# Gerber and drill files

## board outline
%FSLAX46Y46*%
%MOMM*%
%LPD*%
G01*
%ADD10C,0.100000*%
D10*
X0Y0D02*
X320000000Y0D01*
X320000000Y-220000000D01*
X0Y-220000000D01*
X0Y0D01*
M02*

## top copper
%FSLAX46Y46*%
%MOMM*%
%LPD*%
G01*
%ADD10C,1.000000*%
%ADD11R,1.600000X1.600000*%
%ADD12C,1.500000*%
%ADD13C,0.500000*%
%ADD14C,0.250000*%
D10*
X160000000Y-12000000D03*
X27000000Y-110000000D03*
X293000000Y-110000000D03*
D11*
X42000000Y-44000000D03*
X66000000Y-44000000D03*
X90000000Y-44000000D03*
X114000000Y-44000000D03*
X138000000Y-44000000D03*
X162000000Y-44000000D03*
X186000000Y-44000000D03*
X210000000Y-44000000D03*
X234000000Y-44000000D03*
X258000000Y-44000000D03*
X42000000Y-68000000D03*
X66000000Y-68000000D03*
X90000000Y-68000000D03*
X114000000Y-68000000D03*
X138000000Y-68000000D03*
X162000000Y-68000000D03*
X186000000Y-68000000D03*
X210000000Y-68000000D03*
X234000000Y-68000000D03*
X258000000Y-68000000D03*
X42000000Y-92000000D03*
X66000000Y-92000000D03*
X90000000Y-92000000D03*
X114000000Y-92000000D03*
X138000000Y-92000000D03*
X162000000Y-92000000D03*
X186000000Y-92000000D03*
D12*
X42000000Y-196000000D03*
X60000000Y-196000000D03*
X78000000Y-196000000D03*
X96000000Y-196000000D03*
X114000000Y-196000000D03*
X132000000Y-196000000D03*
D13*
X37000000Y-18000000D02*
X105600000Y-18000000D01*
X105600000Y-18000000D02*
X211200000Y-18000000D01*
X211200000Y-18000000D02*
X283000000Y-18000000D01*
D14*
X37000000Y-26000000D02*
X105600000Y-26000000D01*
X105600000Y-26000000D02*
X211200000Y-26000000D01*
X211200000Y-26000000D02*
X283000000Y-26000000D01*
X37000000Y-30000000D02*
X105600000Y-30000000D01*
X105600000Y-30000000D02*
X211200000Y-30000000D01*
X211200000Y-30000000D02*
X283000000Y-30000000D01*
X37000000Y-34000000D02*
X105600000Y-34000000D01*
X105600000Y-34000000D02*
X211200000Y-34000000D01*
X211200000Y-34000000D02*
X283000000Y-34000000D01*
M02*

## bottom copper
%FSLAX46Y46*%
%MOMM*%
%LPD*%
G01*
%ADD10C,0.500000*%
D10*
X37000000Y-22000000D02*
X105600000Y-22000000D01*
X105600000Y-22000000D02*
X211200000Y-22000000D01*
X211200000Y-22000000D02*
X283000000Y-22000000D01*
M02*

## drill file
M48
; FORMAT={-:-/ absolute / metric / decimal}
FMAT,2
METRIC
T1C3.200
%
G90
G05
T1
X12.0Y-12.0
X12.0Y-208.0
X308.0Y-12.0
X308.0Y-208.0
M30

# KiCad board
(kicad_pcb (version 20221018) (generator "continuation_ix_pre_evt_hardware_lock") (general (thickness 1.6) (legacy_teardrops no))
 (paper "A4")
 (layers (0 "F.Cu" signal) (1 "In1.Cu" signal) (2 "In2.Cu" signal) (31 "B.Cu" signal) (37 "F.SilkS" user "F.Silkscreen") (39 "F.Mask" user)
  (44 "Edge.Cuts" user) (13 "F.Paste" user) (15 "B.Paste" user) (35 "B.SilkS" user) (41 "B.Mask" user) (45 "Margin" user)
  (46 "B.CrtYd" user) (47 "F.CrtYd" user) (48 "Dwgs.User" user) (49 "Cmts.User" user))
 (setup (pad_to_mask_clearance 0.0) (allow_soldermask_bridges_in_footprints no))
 (gr_rect (start 0 0) (end 320.0 220.0) (stroke (width 0.1) (type default)) (fill none) (layer "Edge.Cuts"))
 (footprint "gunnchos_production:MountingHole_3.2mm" (layer "F.Cu") (at 12.0 12.0)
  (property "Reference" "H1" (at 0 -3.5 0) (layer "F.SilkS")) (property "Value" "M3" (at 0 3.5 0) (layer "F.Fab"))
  (pad "" np_thru_hole circle (at 0 0) (size 3.2 3.2) (drill 3.2) (layers "*.Cu" "*.Mask")))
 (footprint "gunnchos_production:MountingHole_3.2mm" (layer "F.Cu") (at 308.0 12.0)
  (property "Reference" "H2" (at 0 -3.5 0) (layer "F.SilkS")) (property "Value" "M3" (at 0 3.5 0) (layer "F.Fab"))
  (pad "" np_thru_hole circle (at 0 0) (size 3.2 3.2) (drill 3.2) (layers "*.Cu" "*.Mask")))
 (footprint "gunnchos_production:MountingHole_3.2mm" (layer "F.Cu") (at 12.0 208.0)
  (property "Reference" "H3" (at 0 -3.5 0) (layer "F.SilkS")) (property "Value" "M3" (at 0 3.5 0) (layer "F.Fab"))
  (pad "" np_thru_hole circle (at 0 0) (size 3.2 3.2) (drill 3.2) (layers "*.Cu" "*.Mask")))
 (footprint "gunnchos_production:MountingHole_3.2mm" (layer "F.Cu") (at 308.0 208.0)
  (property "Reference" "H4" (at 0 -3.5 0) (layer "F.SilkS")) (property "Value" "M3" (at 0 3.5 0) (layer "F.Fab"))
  (pad "" np_thru_hole circle (at 0 0) (size 3.2 3.2) (drill 3.2) (layers "*.Cu" "*.Mask")))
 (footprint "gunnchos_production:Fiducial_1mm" (layer "F.Cu") (at 160.0 12.0)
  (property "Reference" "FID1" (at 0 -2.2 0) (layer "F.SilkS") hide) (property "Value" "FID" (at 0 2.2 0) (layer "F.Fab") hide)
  (pad "1" smd circle (at 0 0) (size 1 1) (layers "F.Cu") (solder_mask_margin 0.5)))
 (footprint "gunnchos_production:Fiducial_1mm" (layer "F.Cu") (at 27.0 110.0)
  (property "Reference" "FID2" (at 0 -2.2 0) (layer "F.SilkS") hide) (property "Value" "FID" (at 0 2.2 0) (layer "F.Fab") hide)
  (pad "1" smd circle (at 0 0) (size 1 1) (layers "F.Cu") (solder_mask_margin 0.5)))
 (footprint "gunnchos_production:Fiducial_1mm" (layer "F.Cu") (at 293.0 110.0)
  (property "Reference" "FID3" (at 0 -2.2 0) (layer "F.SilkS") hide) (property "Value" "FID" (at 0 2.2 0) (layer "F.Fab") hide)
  (pad "1" smd circle (at 0 0) (size 1 1) (layers "F.Cu") (solder_mask_margin 0.5)))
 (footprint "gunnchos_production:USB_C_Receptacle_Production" (layer "F.Cu") (at 42.00 44.00)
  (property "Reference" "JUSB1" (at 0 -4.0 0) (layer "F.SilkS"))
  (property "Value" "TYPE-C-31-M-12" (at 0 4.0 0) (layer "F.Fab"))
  (pad "1" smd rect (at 0 0) (size 1.6 1.6) (layers "F.Cu" "F.Paste" "F.Mask")))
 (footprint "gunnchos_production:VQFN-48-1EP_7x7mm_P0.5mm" (layer "F.Cu") (at 66.00 44.00)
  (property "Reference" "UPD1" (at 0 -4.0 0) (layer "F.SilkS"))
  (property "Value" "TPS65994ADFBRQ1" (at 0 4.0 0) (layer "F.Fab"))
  (pad "1" smd rect (at 0 0) (size 1.6 1.6) (layers "F.Cu" "F.Paste" "F.Mask")))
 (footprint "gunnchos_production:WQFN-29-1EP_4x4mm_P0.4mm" (layer "F.Cu") (at 90.00 44.00)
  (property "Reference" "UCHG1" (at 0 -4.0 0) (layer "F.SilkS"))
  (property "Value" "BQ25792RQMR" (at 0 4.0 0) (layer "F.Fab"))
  (pad "1" smd rect (at 0 0) (size 1.6 1.6) (layers "F.Cu" "F.Paste" "F.Mask")))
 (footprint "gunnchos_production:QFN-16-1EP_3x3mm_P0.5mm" (layer "F.Cu") (at 114.00 44.00)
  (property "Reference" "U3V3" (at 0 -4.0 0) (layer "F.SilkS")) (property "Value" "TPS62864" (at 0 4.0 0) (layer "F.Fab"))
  (pad "1" smd rect (at 0 0) (size 1.6 1.6) (layers "F.Cu" "F.Paste" "F.Mask")))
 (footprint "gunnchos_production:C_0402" (layer "F.Cu") (at 138.00 44.00) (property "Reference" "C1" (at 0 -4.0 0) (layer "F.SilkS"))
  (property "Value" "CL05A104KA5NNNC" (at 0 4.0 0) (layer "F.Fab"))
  (pad "1" smd rect (at 0 0) (size 1.6 1.6) (layers "F.Cu" "F.Paste" "F.Mask")))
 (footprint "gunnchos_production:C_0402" (layer "F.Cu") (at 162.00 44.00) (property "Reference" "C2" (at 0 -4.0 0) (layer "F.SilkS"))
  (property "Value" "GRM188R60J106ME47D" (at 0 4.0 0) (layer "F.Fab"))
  (pad "1" smd rect (at 0 0) (size 1.6 1.6) (layers "F.Cu" "F.Paste" "F.Mask")))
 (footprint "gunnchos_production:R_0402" (layer "F.Cu") (at 186.00 44.00) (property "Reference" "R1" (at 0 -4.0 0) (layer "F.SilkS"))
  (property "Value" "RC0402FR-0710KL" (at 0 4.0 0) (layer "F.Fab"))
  (pad "1" smd rect (at 0 0) (size 1.6 1.6) (layers "F.Cu" "F.Paste" "F.Mask")))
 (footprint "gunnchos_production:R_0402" (layer "F.Cu") (at 210.00 44.00) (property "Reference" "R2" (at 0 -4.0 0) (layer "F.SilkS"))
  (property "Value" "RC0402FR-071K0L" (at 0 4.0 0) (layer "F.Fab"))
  (pad "1" smd rect (at 0 0) (size 1.6 1.6) (layers "F.Cu" "F.Paste" "F.Mask")))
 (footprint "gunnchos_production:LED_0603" (layer "F.Cu") (at 234.00 44.00) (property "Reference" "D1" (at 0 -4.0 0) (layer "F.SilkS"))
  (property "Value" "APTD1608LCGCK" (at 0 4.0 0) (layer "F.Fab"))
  (pad "1" smd rect (at 0 0) (size 1.6 1.6) (layers "F.Cu" "F.Paste" "F.Mask")))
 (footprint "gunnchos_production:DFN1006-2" (layer "F.Cu") (at 258.00 44.00)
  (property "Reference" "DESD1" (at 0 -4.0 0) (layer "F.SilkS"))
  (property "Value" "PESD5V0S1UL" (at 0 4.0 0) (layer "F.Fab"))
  (pad "1" smd rect (at 0 0) (size 1.6 1.6) (layers "F.Cu" "F.Paste" "F.Mask")))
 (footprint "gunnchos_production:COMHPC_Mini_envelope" (layer "F.Cu") (at 42.00 68.00)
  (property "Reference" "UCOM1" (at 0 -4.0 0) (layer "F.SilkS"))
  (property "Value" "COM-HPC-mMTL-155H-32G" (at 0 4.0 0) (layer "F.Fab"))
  (pad "1" smd rect (at 0 0) (size 1.6 1.6) (layers "F.Cu" "F.Paste" "F.Mask")))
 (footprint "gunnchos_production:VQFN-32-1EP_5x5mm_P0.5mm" (layer "F.Cu") (at 66.00 68.00)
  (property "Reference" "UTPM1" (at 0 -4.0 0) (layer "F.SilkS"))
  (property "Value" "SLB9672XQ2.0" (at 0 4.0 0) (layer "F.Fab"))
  (pad "1" smd rect (at 0 0) (size 1.6 1.6) (layers "F.Cu" "F.Paste" "F.Mask")))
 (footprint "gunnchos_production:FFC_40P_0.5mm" (layer "F.Cu") (at 90.00 68.00)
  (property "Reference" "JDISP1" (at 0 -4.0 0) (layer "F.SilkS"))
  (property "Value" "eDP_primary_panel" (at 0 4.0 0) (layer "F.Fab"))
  (pad "1" smd rect (at 0 0) (size 1.6 1.6) (layers "F.Cu" "F.Paste" "F.Mask")))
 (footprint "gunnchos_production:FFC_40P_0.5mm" (layer "F.Cu") (at 114.00 68.00)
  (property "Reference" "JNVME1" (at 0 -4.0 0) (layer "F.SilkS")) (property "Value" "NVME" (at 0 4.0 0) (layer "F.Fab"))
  (pad "1" smd rect (at 0 0) (size 1.6 1.6) (layers "F.Cu" "F.Paste" "F.Mask")))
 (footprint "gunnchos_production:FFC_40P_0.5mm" (layer "F.Cu") (at 138.00 68.00)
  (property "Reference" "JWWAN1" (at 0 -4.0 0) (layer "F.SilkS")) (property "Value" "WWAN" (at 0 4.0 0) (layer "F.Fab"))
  (pad "1" smd rect (at 0 0) (size 1.6 1.6) (layers "F.Cu" "F.Paste" "F.Mask")))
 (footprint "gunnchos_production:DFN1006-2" (layer "F.Cu") (at 162.00 68.00)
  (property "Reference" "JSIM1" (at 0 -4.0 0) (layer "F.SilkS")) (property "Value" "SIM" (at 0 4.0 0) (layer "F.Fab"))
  (pad "1" smd rect (at 0 0) (size 1.6 1.6) (layers "F.Cu" "F.Paste" "F.Mask")))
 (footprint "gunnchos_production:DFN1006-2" (layer "F.Cu") (at 186.00 68.00)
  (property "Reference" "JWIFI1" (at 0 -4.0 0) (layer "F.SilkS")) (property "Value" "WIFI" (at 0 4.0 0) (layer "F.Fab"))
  (pad "1" smd rect (at 0 0) (size 1.6 1.6) (layers "F.Cu" "F.Paste" "F.Mask")))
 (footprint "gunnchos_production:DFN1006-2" (layer "F.Cu") (at 210.00 68.00)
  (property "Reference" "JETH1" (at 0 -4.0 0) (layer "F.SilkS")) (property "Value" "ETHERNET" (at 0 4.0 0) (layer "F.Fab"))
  (pad "1" smd rect (at 0 0) (size 1.6 1.6) (layers "F.Cu" "F.Paste" "F.Mask")))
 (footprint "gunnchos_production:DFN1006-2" (layer "F.Cu") (at 234.00 68.00)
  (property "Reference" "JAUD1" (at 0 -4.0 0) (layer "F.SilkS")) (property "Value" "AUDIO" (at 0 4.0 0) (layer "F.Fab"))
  (pad "1" smd rect (at 0 0) (size 1.6 1.6) (layers "F.Cu" "F.Paste" "F.Mask")))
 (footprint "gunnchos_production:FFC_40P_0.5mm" (layer "F.Cu") (at 258.00 68.00)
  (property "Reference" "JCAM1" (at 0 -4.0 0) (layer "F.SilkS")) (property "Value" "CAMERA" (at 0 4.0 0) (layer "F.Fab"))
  (pad "1" smd rect (at 0 0) (size 1.6 1.6) (layers "F.Cu" "F.Paste" "F.Mask")))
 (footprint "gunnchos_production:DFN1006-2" (layer "F.Cu") (at 42.00 92.00)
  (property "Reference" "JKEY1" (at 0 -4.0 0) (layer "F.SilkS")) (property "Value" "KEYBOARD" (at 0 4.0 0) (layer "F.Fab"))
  (pad "1" smd rect (at 0 0) (size 1.6 1.6) (layers "F.Cu" "F.Paste" "F.Mask")))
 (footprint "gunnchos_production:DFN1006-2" (layer "F.Cu") (at 66.00 92.00)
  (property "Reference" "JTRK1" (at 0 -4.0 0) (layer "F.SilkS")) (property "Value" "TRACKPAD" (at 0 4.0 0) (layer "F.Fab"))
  (pad "1" smd rect (at 0 0) (size 1.6 1.6) (layers "F.Cu" "F.Paste" "F.Mask")))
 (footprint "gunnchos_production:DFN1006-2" (layer "F.Cu") (at 90.00 92.00)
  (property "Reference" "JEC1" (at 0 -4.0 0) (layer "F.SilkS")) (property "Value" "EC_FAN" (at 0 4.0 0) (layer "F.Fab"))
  (pad "1" smd rect (at 0 0) (size 1.6 1.6) (layers "F.Cu" "F.Paste" "F.Mask")))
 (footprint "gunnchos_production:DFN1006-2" (layer "F.Cu") (at 114.00 92.00)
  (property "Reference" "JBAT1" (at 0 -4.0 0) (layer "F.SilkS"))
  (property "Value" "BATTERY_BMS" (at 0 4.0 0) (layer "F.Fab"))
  (pad "1" smd rect (at 0 0) (size 1.6 1.6) (layers "F.Cu" "F.Paste" "F.Mask")))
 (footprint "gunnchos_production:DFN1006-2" (layer "F.Cu") (at 138.00 92.00)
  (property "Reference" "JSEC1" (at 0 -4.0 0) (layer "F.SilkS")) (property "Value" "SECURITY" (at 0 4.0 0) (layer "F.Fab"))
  (pad "1" smd rect (at 0 0) (size 1.6 1.6) (layers "F.Cu" "F.Paste" "F.Mask")))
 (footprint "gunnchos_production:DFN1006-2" (layer "F.Cu") (at 162.00 92.00)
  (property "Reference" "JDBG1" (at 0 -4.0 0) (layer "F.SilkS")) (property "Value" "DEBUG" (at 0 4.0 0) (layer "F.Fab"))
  (pad "1" smd rect (at 0 0) (size 1.6 1.6) (layers "F.Cu" "F.Paste" "F.Mask")))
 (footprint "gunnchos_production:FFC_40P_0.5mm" (layer "F.Cu") (at 186.00 92.00)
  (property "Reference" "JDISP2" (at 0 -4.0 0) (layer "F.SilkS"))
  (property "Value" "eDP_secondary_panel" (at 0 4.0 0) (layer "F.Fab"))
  (pad "1" smd rect (at 0 0) (size 1.6 1.6) (layers "F.Cu" "F.Paste" "F.Mask")))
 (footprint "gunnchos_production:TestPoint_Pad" (layer "F.Cu") (at 42.0 196.0) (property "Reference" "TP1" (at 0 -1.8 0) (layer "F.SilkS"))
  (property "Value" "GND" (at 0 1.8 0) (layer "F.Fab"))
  (pad "1" smd circle (at 0 0) (size 1.5 1.5) (layers "F.Cu" "F.Mask")))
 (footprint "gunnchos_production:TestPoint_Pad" (layer "F.Cu") (at 60.0 196.0) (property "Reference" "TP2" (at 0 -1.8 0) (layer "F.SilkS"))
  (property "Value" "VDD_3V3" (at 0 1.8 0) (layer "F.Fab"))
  (pad "1" smd circle (at 0 0) (size 1.5 1.5) (layers "F.Cu" "F.Mask")))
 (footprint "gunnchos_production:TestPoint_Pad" (layer "F.Cu") (at 78.0 196.0) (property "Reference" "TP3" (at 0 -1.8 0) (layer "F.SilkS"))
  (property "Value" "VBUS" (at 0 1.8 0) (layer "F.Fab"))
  (pad "1" smd circle (at 0 0) (size 1.5 1.5) (layers "F.Cu" "F.Mask")))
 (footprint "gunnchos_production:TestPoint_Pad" (layer "F.Cu") (at 96.0 196.0) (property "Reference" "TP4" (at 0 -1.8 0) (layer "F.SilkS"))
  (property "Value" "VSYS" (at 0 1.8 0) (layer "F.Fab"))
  (pad "1" smd circle (at 0 0) (size 1.5 1.5) (layers "F.Cu" "F.Mask")))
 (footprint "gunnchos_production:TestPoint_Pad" (layer "F.Cu") (at 114.0 196.0) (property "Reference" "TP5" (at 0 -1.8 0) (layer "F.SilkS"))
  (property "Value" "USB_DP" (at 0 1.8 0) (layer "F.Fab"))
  (pad "1" smd circle (at 0 0) (size 1.5 1.5) (layers "F.Cu" "F.Mask")))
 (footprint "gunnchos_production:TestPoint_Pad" (layer "F.Cu") (at 132.0 196.0) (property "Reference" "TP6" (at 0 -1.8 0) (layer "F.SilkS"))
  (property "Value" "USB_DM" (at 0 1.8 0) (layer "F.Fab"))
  (pad "1" smd circle (at 0 0) (size 1.5 1.5) (layers "F.Cu" "F.Mask")))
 (segment (start 37.00 18.00) (end 105.60 18.00) (width 0.5) (layer "F.Cu") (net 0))
 (segment (start 105.60 18.00) (end 211.20 18.00) (width 0.5) (layer "F.Cu") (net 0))
 (segment (start 211.20 18.00) (end 283.00 18.00) (width 0.5) (layer "F.Cu") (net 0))
 (segment (start 37.00 22.00) (end 105.60 22.00) (width 0.5) (layer "B.Cu") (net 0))
 (segment (start 105.60 22.00) (end 211.20 22.00) (width 0.5) (layer "B.Cu") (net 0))
 (segment (start 211.20 22.00) (end 283.00 22.00) (width 0.5) (layer "B.Cu") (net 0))
 (segment (start 37.00 26.00) (end 105.60 26.00) (width 0.25) (layer "F.Cu") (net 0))
 (segment (start 105.60 26.00) (end 211.20 26.00) (width 0.25) (layer "F.Cu") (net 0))
 (segment (start 211.20 26.00) (end 283.00 26.00) (width 0.25) (layer "F.Cu") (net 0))
 (segment (start 37.00 30.00) (end 105.60 30.00) (width 0.25) (layer "F.Cu") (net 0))
 (segment (start 105.60 30.00) (end 211.20 30.00) (width 0.25) (layer "F.Cu") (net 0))
 (segment (start 211.20 30.00) (end 283.00 30.00) (width 0.25) (layer "F.Cu") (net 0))
 (segment (start 37.00 34.00) (end 105.60 34.00) (width 0.25) (layer "F.Cu") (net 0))
 (segment (start 105.60 34.00) (end 211.20 34.00) (width 0.25) (layer "F.Cu") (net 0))
 (segment (start 211.20 34.00) (end 283.00 34.00) (width 0.25) (layer "F.Cu") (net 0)))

